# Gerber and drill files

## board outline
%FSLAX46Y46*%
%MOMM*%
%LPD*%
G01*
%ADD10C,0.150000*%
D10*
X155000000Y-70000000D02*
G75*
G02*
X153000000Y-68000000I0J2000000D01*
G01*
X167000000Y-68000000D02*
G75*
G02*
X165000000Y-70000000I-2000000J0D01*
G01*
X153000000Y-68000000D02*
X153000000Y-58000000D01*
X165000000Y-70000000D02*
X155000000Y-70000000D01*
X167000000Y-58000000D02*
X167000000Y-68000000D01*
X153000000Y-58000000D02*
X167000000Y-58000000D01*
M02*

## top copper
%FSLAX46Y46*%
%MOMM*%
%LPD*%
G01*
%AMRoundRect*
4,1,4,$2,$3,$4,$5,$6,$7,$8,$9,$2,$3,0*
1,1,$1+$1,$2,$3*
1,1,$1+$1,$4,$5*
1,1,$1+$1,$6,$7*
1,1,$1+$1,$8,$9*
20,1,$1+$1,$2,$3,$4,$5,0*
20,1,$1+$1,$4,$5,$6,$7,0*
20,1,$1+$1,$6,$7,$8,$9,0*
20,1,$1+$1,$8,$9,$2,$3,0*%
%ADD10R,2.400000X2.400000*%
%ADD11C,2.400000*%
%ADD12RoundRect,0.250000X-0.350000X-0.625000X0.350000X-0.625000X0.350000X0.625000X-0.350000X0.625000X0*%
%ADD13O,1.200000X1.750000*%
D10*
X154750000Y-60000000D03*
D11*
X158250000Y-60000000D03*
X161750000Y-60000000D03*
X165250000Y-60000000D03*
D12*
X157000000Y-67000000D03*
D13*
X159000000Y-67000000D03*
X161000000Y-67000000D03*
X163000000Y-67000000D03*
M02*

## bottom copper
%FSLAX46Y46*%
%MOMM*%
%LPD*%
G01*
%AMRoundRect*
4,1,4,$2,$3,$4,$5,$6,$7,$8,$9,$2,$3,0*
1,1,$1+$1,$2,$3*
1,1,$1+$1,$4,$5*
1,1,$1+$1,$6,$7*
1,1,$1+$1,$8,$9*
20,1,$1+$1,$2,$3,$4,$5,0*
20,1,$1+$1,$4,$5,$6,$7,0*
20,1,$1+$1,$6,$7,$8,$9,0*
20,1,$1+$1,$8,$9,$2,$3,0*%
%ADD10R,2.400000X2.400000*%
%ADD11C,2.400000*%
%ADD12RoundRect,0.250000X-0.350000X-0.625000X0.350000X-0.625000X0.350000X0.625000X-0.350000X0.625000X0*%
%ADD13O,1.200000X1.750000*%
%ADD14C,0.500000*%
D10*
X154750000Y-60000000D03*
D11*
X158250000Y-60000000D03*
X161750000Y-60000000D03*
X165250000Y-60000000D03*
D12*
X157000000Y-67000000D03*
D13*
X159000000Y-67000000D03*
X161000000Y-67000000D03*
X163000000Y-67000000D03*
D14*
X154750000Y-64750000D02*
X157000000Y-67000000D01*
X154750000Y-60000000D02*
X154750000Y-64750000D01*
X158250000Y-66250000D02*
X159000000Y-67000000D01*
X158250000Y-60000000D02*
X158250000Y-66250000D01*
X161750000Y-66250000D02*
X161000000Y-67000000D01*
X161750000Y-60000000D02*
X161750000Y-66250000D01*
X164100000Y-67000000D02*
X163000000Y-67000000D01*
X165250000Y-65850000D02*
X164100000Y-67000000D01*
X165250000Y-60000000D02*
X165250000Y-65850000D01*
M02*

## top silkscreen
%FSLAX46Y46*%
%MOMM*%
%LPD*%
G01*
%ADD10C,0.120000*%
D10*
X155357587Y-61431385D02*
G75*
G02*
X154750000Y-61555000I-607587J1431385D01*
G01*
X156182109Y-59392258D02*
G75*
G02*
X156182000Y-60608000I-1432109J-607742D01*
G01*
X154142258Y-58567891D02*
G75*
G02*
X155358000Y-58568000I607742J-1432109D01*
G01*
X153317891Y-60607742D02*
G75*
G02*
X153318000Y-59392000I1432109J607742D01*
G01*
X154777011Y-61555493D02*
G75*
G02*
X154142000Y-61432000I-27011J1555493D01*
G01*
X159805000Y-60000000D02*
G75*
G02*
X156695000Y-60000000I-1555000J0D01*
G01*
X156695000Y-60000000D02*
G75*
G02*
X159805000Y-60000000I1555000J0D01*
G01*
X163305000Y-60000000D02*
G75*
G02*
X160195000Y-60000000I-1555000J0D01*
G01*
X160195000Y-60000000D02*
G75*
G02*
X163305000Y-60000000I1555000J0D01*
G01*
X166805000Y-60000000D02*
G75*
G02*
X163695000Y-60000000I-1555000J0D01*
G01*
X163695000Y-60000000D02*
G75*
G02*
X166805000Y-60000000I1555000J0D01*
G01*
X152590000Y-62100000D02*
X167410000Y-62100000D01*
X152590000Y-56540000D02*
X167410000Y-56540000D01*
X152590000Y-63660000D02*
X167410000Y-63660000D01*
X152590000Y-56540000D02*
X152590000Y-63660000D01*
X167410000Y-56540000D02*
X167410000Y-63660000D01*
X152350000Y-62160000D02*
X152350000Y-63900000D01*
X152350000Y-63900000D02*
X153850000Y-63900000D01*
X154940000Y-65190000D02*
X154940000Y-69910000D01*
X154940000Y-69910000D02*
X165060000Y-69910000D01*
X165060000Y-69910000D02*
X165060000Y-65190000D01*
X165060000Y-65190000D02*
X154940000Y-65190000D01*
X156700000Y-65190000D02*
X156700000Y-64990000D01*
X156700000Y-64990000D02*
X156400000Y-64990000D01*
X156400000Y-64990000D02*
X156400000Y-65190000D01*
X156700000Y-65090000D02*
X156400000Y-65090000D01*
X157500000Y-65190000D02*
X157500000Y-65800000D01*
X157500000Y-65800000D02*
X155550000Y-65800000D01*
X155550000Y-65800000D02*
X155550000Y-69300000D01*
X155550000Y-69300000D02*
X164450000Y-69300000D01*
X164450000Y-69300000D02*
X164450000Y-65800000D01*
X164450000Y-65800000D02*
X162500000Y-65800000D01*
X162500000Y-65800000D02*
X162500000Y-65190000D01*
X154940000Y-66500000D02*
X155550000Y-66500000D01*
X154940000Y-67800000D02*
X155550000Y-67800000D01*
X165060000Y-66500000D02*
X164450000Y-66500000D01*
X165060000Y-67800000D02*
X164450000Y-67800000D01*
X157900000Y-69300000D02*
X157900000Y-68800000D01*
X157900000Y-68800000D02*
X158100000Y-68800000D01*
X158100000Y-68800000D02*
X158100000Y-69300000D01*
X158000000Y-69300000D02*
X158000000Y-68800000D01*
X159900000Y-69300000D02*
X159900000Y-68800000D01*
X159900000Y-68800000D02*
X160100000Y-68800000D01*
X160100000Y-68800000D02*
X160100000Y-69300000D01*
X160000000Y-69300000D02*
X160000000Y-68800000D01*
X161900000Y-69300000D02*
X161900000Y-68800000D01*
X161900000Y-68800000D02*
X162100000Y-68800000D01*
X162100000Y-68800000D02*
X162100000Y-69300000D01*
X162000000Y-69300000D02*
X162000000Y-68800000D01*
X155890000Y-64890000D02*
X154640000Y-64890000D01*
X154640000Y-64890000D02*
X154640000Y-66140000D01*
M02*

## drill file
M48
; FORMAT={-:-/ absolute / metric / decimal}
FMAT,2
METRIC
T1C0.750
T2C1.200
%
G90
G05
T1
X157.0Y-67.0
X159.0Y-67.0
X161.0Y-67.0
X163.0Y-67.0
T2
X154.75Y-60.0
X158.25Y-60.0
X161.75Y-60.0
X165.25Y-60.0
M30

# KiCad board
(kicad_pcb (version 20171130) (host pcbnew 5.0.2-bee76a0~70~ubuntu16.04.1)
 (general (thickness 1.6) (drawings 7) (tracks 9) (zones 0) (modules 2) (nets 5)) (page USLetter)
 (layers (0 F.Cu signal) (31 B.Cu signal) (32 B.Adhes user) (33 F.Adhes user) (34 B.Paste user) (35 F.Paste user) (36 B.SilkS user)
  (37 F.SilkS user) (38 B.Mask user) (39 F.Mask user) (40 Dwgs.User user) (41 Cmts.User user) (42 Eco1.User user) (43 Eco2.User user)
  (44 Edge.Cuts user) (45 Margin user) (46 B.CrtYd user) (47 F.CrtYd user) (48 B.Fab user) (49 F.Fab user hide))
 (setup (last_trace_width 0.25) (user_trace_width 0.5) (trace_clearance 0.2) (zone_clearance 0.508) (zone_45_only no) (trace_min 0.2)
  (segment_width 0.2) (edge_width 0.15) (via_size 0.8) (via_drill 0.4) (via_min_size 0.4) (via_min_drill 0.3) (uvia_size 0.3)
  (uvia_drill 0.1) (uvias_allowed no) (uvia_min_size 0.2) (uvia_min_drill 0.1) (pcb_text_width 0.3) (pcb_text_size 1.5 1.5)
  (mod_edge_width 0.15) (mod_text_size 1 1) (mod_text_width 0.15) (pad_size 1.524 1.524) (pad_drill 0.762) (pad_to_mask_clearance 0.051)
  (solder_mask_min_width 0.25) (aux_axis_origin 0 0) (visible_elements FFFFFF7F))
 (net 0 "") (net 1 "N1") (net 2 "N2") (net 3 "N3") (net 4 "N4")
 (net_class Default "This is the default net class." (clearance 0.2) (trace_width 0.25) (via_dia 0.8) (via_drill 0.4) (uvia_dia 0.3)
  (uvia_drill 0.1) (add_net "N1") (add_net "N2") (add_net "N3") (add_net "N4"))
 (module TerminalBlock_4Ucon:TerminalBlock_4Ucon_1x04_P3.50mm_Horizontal (layer F.Cu) (at 154.75 60)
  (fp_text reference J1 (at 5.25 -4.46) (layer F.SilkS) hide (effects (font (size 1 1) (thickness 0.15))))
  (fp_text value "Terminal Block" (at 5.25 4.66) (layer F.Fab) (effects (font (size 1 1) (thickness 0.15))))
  (fp_arc (start 0 0) (end 0 1.555) (angle -23) (layer F.SilkS) (width 0.12))
  (fp_arc (start 0 0) (end 1.432 0.608) (angle -46) (layer F.SilkS) (width 0.12))
  (fp_arc (start 0 0) (end 0.608 -1.432) (angle -46) (layer F.SilkS) (width 0.12))
  (fp_arc (start 0 0) (end -1.432 -0.608) (angle -46) (layer F.SilkS) (width 0.12))
  (fp_arc (start 0 0) (end -0.608 1.432) (angle -24) (layer F.SilkS) (width 0.12))
  (fp_circle (center 3.5 0) (end 5.055 0) (layer F.SilkS) (width 0.12))
  (fp_circle (center 7 0) (end 8.555 0) (layer F.SilkS) (width 0.12))
  (fp_circle (center 10.5 0) (end 12.055 0) (layer F.SilkS) (width 0.12))
  (fp_line (start -2.16 2.1) (end 12.66 2.1) (layer F.SilkS) (width 0.12))
  (fp_line (start -2.16 -3.46) (end 12.66 -3.46) (layer F.SilkS) (width 0.12))
  (fp_line (start -2.16 3.66) (end 12.66 3.66) (layer F.SilkS) (width 0.12))
  (fp_line (start -2.16 -3.46) (end -2.16 3.66) (layer F.SilkS) (width 0.12))
  (fp_line (start 12.66 -3.46) (end 12.66 3.66) (layer F.SilkS) (width 0.12))
  (fp_line (start -2.4 2.16) (end -2.4 3.9) (layer F.SilkS) (width 0.12))
  (fp_line (start -2.4 3.9) (end -0.9 3.9) (layer F.SilkS) (width 0.12))
  (pad 1 thru_hole rect (at 0 0) (size 2.4 2.4) (drill 1.2) (layers *.Cu *.Mask) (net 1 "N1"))
  (pad 2 thru_hole circle (at 3.5 0) (size 2.4 2.4) (drill 1.2) (layers *.Cu *.Mask) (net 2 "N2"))
  (pad 3 thru_hole circle (at 7 0) (size 2.4 2.4) (drill 1.2) (layers *.Cu *.Mask) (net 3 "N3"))
  (pad 4 thru_hole circle (at 10.5 0) (size 2.4 2.4) (drill 1.2) (layers *.Cu *.Mask) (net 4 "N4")))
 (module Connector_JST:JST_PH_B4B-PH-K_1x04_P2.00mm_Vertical (layer F.Cu) (at 157 67)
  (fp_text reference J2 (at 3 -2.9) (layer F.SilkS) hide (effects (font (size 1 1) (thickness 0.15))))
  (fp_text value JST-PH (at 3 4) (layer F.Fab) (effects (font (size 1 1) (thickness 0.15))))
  (fp_line (start -2.06 -1.81) (end -2.06 2.91) (layer F.SilkS) (width 0.12))
  (fp_line (start -2.06 2.91) (end 8.06 2.91) (layer F.SilkS) (width 0.12))
  (fp_line (start 8.06 2.91) (end 8.06 -1.81) (layer F.SilkS) (width 0.12))
  (fp_line (start 8.06 -1.81) (end -2.06 -1.81) (layer F.SilkS) (width 0.12))
  (fp_line (start -0.3 -1.81) (end -0.3 -2.01) (layer F.SilkS) (width 0.12))
  (fp_line (start -0.3 -2.01) (end -0.6 -2.01) (layer F.SilkS) (width 0.12))
  (fp_line (start -0.6 -2.01) (end -0.6 -1.81) (layer F.SilkS) (width 0.12))
  (fp_line (start -0.3 -1.91) (end -0.6 -1.91) (layer F.SilkS) (width 0.12))
  (fp_line (start 0.5 -1.81) (end 0.5 -1.2) (layer F.SilkS) (width 0.12))
  (fp_line (start 0.5 -1.2) (end -1.45 -1.2) (layer F.SilkS) (width 0.12))
  (fp_line (start -1.45 -1.2) (end -1.45 2.3) (layer F.SilkS) (width 0.12))
  (fp_line (start -1.45 2.3) (end 7.45 2.3) (layer F.SilkS) (width 0.12))
  (fp_line (start 7.45 2.3) (end 7.45 -1.2) (layer F.SilkS) (width 0.12))
  (fp_line (start 7.45 -1.2) (end 5.5 -1.2) (layer F.SilkS) (width 0.12))
  (fp_line (start 5.5 -1.2) (end 5.5 -1.81) (layer F.SilkS) (width 0.12))
  (fp_line (start -2.06 -0.5) (end -1.45 -0.5) (layer F.SilkS) (width 0.12))
  (fp_line (start -2.06 0.8) (end -1.45 0.8) (layer F.SilkS) (width 0.12))
  (fp_line (start 8.06 -0.5) (end 7.45 -0.5) (layer F.SilkS) (width 0.12))
  (fp_line (start 8.06 0.8) (end 7.45 0.8) (layer F.SilkS) (width 0.12))
  (fp_line (start 0.9 2.3) (end 0.9 1.8) (layer F.SilkS) (width 0.12))
  (fp_line (start 0.9 1.8) (end 1.1 1.8) (layer F.SilkS) (width 0.12))
  (fp_line (start 1.1 1.8) (end 1.1 2.3) (layer F.SilkS) (width 0.12))
  (fp_line (start 1 2.3) (end 1 1.8) (layer F.SilkS) (width 0.12))
  (fp_line (start 2.9 2.3) (end 2.9 1.8) (layer F.SilkS) (width 0.12))
  (fp_line (start 2.9 1.8) (end 3.1 1.8) (layer F.SilkS) (width 0.12))
  (fp_line (start 3.1 1.8) (end 3.1 2.3) (layer F.SilkS) (width 0.12))
  (fp_line (start 3 2.3) (end 3 1.8) (layer F.SilkS) (width 0.12))
  (fp_line (start 4.9 2.3) (end 4.9 1.8) (layer F.SilkS) (width 0.12))
  (fp_line (start 4.9 1.8) (end 5.1 1.8) (layer F.SilkS) (width 0.12))
  (fp_line (start 5.1 1.8) (end 5.1 2.3) (layer F.SilkS) (width 0.12))
  (fp_line (start 5 2.3) (end 5 1.8) (layer F.SilkS) (width 0.12))
  (fp_line (start -1.11 -2.11) (end -2.36 -2.11) (layer F.SilkS) (width 0.12))
  (fp_line (start -2.36 -2.11) (end -2.36 -0.86) (layer F.SilkS) (width 0.12))
  (pad 1 thru_hole roundrect (at 0 0) (size 1.2 1.75) (drill 0.75) (layers *.Cu *.Mask) (roundrect_rratio 0.208333) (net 1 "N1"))
  (pad 2 thru_hole oval (at 2 0) (size 1.2 1.75) (drill 0.75) (layers *.Cu *.Mask) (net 2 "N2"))
  (pad 3 thru_hole oval (at 4 0) (size 1.2 1.75) (drill 0.75) (layers *.Cu *.Mask) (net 3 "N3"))
  (pad 4 thru_hole oval (at 6 0) (size 1.2 1.75) (drill 0.75) (layers *.Cu *.Mask) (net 4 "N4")))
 (gr_arc (start 155 68) (end 153 68) (angle -90) (layer Edge.Cuts) (width 0.15))
 (gr_arc (start 165 68) (end 165 70) (angle -90) (layer Edge.Cuts) (width 0.15))
 (gr_line (start 153 68) (end 153 58) (layer Edge.Cuts) (width 0.15))
 (gr_line (start 165 70) (end 155 70) (layer Edge.Cuts) (width 0.15))
 (gr_line (start 167 58) (end 167 68) (layer Edge.Cuts) (width 0.15))
 (gr_line (start 153 58) (end 167 58) (layer Edge.Cuts) (width 0.15))
 (segment (start 154.75 64.75) (end 157 67) (width 0.5) (layer B.Cu) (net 1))
 (segment (start 154.75 60) (end 154.75 64.75) (width 0.5) (layer B.Cu) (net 1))
 (segment (start 158.25 66.25) (end 159 67) (width 0.5) (layer B.Cu) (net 2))
 (segment (start 158.25 60) (end 158.25 66.25) (width 0.5) (layer B.Cu) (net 2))
 (segment (start 161.75 66.25) (end 161 67) (width 0.5) (layer B.Cu) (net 3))
 (segment (start 161.75 60) (end 161.75 66.25) (width 0.5) (layer B.Cu) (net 3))
 (segment (start 164.1 67) (end 163 67) (width 0.5) (layer B.Cu) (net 4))
 (segment (start 165.25 65.85) (end 164.1 67) (width 0.5) (layer B.Cu) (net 4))
 (segment (start 165.25 60) (end 165.25 65.85) (width 0.5) (layer B.Cu) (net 4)))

